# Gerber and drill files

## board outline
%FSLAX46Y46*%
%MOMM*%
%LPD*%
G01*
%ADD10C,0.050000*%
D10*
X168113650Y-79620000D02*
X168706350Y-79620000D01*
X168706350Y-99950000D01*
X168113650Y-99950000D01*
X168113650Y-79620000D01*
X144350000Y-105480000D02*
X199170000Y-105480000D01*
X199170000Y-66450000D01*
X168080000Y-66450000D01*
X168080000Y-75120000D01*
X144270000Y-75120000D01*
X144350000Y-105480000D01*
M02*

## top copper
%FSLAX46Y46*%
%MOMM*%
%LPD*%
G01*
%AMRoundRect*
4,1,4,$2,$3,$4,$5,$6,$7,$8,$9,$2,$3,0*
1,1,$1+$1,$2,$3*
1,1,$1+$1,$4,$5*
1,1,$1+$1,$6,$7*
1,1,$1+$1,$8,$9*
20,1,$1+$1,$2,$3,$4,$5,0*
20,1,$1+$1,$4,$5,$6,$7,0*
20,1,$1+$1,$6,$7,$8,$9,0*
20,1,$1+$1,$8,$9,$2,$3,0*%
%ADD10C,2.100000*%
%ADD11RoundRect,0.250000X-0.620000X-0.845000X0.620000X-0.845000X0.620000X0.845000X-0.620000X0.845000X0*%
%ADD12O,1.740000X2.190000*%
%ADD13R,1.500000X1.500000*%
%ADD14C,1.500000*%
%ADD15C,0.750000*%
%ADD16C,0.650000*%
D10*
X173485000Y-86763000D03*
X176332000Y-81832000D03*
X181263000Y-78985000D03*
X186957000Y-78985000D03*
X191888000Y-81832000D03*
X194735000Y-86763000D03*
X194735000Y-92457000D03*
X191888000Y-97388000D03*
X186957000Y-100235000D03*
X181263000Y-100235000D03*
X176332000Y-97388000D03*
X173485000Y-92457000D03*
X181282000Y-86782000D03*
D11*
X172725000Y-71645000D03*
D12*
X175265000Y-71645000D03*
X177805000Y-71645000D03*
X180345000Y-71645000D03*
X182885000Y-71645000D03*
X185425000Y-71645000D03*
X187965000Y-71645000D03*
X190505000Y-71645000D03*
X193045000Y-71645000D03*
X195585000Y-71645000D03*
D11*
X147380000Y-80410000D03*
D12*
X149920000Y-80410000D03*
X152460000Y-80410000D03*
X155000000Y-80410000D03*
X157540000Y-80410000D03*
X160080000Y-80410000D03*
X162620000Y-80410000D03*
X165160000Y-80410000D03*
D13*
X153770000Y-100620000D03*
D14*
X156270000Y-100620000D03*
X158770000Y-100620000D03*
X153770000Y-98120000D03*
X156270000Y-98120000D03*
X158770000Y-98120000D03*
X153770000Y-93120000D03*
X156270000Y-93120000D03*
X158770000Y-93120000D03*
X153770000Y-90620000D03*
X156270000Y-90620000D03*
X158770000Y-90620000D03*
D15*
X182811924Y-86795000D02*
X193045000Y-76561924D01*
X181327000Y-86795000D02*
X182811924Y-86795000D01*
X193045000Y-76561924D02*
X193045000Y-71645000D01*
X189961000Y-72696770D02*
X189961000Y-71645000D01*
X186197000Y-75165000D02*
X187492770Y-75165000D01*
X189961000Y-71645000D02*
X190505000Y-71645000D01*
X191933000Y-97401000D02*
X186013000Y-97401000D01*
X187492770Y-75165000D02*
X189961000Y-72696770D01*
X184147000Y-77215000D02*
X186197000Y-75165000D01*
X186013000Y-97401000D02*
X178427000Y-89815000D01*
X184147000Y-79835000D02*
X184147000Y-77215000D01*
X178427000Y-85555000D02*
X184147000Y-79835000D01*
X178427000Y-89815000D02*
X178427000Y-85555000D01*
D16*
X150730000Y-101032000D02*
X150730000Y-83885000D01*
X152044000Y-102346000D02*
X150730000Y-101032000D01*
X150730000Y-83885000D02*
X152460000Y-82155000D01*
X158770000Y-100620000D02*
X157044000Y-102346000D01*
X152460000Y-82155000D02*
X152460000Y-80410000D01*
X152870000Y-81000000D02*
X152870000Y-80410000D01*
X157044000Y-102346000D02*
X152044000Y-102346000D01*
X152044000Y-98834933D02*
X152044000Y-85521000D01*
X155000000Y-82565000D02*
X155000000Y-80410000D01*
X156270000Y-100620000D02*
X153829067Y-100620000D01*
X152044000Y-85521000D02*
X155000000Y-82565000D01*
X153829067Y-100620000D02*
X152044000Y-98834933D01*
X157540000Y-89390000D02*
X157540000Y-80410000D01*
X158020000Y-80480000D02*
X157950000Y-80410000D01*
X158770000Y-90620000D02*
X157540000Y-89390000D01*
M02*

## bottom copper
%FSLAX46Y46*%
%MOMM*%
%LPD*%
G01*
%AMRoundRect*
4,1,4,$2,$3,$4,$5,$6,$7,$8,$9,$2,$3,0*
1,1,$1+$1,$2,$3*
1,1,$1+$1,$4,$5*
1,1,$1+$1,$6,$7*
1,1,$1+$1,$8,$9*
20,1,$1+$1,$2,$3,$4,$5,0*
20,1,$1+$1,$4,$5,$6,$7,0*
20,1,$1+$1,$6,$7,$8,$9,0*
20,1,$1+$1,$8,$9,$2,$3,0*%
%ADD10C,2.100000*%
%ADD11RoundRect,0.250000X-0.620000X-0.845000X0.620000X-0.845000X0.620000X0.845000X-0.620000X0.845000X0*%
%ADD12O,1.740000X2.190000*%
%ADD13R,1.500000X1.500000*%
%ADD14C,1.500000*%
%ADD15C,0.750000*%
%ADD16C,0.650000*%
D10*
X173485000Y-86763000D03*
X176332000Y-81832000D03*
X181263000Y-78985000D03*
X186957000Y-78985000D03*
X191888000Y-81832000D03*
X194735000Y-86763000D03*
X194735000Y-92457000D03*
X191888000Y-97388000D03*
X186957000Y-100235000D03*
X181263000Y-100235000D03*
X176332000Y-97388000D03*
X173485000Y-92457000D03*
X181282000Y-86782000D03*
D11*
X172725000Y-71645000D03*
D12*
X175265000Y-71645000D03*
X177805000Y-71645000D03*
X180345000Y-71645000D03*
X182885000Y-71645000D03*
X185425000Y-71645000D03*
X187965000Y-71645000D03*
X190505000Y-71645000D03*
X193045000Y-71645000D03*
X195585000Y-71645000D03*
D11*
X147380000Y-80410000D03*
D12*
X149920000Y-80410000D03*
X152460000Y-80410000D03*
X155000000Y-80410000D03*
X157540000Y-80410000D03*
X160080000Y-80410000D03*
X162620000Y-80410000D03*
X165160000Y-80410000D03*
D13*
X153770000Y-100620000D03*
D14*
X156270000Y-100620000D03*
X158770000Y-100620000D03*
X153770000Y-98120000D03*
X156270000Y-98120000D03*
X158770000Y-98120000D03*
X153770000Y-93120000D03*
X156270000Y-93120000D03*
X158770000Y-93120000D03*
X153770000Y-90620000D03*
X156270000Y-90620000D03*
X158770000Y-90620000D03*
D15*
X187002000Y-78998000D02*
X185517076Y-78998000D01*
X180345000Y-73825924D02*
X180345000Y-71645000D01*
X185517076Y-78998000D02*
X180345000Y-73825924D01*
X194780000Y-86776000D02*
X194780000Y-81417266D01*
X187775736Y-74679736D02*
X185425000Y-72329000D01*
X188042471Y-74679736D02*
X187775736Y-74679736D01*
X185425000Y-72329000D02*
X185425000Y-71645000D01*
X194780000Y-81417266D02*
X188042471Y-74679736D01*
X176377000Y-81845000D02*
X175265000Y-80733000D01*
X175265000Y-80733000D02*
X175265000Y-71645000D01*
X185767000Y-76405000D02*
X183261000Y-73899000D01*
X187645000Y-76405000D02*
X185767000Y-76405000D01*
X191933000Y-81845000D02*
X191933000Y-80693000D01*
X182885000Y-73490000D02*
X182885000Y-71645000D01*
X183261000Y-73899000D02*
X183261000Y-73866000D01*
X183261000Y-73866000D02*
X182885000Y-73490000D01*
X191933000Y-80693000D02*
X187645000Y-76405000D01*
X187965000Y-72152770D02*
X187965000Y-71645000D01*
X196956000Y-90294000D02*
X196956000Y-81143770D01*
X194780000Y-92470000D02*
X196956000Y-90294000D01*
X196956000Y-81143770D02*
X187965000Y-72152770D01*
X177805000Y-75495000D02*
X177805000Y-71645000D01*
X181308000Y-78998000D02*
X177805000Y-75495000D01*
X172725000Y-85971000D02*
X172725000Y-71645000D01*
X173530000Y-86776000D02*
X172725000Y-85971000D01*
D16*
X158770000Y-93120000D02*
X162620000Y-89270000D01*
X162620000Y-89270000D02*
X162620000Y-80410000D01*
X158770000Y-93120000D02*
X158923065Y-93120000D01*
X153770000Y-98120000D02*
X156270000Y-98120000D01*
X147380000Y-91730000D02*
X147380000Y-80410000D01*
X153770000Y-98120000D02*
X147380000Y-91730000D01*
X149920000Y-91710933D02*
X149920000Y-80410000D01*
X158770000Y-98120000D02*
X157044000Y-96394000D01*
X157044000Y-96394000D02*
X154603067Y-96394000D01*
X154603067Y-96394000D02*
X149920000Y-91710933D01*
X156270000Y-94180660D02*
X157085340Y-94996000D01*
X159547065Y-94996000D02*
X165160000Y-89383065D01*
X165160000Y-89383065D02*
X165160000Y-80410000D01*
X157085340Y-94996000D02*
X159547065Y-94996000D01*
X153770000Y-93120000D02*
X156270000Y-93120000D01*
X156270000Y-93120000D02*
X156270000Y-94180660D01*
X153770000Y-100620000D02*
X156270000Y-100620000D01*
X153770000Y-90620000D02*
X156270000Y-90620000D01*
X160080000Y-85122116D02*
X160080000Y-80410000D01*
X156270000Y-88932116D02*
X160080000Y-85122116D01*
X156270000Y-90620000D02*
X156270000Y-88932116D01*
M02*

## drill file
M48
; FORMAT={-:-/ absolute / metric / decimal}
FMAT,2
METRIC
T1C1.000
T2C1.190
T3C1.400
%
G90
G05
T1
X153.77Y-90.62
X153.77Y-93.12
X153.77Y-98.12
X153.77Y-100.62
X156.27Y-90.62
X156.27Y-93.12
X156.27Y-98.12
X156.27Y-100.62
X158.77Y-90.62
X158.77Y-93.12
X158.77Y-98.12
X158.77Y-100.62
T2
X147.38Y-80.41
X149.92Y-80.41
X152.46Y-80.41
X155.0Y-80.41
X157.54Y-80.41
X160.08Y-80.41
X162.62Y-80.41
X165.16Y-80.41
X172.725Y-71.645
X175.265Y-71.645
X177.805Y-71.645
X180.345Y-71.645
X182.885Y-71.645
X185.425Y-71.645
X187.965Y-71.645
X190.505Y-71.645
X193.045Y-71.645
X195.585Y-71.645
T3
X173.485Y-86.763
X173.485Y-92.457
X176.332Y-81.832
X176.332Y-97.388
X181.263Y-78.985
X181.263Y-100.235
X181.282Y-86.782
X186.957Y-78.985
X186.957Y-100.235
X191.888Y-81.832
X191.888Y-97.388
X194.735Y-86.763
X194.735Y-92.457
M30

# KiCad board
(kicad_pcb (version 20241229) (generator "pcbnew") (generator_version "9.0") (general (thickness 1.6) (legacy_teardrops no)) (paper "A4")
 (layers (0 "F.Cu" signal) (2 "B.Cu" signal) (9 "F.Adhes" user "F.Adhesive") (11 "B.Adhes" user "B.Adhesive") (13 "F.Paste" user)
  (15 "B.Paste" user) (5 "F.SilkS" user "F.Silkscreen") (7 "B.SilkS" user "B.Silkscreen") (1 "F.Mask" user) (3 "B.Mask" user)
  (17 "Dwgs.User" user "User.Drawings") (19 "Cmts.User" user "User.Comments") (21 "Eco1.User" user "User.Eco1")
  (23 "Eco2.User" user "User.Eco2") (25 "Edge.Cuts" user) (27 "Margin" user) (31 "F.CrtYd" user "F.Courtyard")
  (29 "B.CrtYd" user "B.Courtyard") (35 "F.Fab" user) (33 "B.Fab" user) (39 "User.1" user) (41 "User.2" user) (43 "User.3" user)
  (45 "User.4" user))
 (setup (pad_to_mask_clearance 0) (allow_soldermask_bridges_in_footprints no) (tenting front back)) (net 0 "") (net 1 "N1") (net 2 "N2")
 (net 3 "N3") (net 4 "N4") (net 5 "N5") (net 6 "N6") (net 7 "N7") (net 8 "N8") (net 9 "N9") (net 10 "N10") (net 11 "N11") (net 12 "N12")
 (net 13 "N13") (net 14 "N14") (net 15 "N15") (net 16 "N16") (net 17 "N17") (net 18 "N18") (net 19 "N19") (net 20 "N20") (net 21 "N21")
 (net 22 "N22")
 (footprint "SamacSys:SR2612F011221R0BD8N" (layer "F.Cu") (at 173.485 86.763)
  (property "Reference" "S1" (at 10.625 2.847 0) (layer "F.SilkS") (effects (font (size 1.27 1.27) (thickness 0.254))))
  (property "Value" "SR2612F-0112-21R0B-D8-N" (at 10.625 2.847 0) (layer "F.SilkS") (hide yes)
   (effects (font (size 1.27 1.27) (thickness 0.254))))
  (pad "1" thru_hole circle (at 0 0) (size 2.1 2.1) (drill 1.4) (layers "*.Cu" "*.Mask") (remove_unused_layers no) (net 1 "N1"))
  (pad "2" thru_hole circle (at 2.847 -4.931) (size 2.1 2.1) (drill 1.4) (layers "*.Cu" "*.Mask") (remove_unused_layers no) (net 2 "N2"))
  (pad "3" thru_hole circle (at 7.778 -7.778) (size 2.1 2.1) (drill 1.4) (layers "*.Cu" "*.Mask") (remove_unused_layers no) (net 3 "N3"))
  (pad "4" thru_hole circle (at 13.472 -7.778) (size 2.1 2.1) (drill 1.4) (layers "*.Cu" "*.Mask") (remove_unused_layers no) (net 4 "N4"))
  (pad "5" thru_hole circle (at 18.403 -4.931) (size 2.1 2.1) (drill 1.4) (layers "*.Cu" "*.Mask") (remove_unused_layers no) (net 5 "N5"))
  (pad "6" thru_hole circle (at 21.25 0) (size 2.1 2.1) (drill 1.4) (layers "*.Cu" "*.Mask") (remove_unused_layers no) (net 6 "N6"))
  (pad "7" thru_hole circle (at 21.25 5.694) (size 2.1 2.1) (drill 1.4) (layers "*.Cu" "*.Mask") (remove_unused_layers no) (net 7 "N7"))
  (pad "8" thru_hole circle (at 18.403 10.625) (size 2.1 2.1) (drill 1.4) (layers "*.Cu" "*.Mask") (remove_unused_layers no) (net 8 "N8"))
  (pad "9" thru_hole circle (at 13.472 13.472) (size 2.1 2.1) (drill 1.4) (layers "*.Cu" "*.Mask") (remove_unused_layers no) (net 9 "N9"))
  (pad "10" thru_hole circle (at 7.778 13.472) (size 2.1 2.1) (drill 1.4) (layers "*.Cu" "*.Mask") (remove_unused_layers no) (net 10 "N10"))
  (pad "11" thru_hole circle (at 2.847 10.625) (size 2.1 2.1) (drill 1.4) (layers "*.Cu" "*.Mask") (remove_unused_layers no) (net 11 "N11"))
  (pad "12" thru_hole circle (at 0 5.694) (size 2.1 2.1) (drill 1.4) (layers "*.Cu" "*.Mask") (remove_unused_layers no) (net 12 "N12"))
  (pad "A1" thru_hole circle (at 7.797 0.019) (size 2.1 2.1) (drill 1.4) (layers "*.Cu" "*.Mask") (remove_unused_layers no) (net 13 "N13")))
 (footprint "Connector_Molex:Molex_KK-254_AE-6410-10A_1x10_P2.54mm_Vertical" (layer "F.Cu") (at 172.725 71.645)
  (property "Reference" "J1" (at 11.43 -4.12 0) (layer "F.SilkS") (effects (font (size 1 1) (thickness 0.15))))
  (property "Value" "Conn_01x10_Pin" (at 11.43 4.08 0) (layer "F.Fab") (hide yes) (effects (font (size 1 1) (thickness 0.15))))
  (pad "1" thru_hole roundrect (at 0 0) (size 1.74 2.19) (drill 1.19) (layers "*.Cu" "*.Mask") (remove_unused_layers no)
   (roundrect_rratio 0.143678) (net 1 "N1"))
  (pad "2" thru_hole oval (at 2.54 0) (size 1.74 2.19) (drill 1.19) (layers "*.Cu" "*.Mask") (remove_unused_layers no) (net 2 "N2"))
  (pad "3" thru_hole oval (at 5.08 0) (size 1.74 2.19) (drill 1.19) (layers "*.Cu" "*.Mask") (remove_unused_layers no) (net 3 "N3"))
  (pad "4" thru_hole oval (at 7.62 0) (size 1.74 2.19) (drill 1.19) (layers "*.Cu" "*.Mask") (remove_unused_layers no) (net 4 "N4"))
  (pad "5" thru_hole oval (at 10.16 0) (size 1.74 2.19) (drill 1.19) (layers "*.Cu" "*.Mask") (remove_unused_layers no) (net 5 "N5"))
  (pad "6" thru_hole oval (at 12.7 0) (size 1.74 2.19) (drill 1.19) (layers "*.Cu" "*.Mask") (remove_unused_layers no) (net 6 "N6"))
  (pad "7" thru_hole oval (at 15.24 0) (size 1.74 2.19) (drill 1.19) (layers "*.Cu" "*.Mask") (remove_unused_layers no) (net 7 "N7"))
  (pad "8" thru_hole oval (at 17.78 0) (size 1.74 2.19) (drill 1.19) (layers "*.Cu" "*.Mask") (remove_unused_layers no) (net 8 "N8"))
  (pad "9" thru_hole oval (at 20.32 0) (size 1.74 2.19) (drill 1.19) (layers "*.Cu" "*.Mask") (remove_unused_layers no) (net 13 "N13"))
  (pad "10" thru_hole oval (at 22.86 0) (size 1.74 2.19) (drill 1.19) (layers "*.Cu" "*.Mask") (remove_unused_layers no) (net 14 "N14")))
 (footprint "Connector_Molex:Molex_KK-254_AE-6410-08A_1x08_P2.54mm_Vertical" (layer "F.Cu") (at 147.38 80.41)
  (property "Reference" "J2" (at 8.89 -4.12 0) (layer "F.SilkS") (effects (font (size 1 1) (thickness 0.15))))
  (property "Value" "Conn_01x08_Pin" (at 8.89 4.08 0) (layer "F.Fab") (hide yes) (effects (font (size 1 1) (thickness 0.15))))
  (pad "1" thru_hole roundrect (at 0 0) (size 1.74 2.19) (drill 1.19) (layers "*.Cu" "*.Mask") (remove_unused_layers no)
   (roundrect_rratio 0.143678) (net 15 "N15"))
  (pad "2" thru_hole oval (at 2.54 0) (size 1.74 2.19) (drill 1.19) (layers "*.Cu" "*.Mask") (remove_unused_layers no) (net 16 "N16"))
  (pad "3" thru_hole oval (at 5.08 0) (size 1.74 2.19) (drill 1.19) (layers "*.Cu" "*.Mask") (remove_unused_layers no) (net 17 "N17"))
  (pad "4" thru_hole oval (at 7.62 0) (size 1.74 2.19) (drill 1.19) (layers "*.Cu" "*.Mask") (remove_unused_layers no) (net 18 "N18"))
  (pad "5" thru_hole oval (at 10.16 0) (size 1.74 2.19) (drill 1.19) (layers "*.Cu" "*.Mask") (remove_unused_layers no) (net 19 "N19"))
  (pad "6" thru_hole oval (at 12.7 0) (size 1.74 2.19) (drill 1.19) (layers "*.Cu" "*.Mask") (remove_unused_layers no) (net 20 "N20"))
  (pad "7" thru_hole oval (at 15.24 0) (size 1.74 2.19) (drill 1.19) (layers "*.Cu" "*.Mask") (remove_unused_layers no) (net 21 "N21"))
  (pad "8" thru_hole oval (at 17.78 0) (size 1.74 2.19) (drill 1.19) (layers "*.Cu" "*.Mask") (remove_unused_layers no) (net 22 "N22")))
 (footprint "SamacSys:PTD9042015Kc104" (layer "F.Cu") (at 153.77 100.62 -90)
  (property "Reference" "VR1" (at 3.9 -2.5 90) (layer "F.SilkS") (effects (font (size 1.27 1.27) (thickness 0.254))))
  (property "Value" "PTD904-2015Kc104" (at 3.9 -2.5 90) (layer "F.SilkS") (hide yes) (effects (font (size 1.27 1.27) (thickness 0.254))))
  (pad "R11" thru_hole rect (at 0 0 270) (size 1.5 1.5) (drill 1) (layers "*.Cu" "*.Mask") (remove_unused_layers no) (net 18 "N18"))
  (pad "R12" thru_hole circle (at 0 -2.5 270) (size 1.5 1.5) (drill 1) (layers "*.Cu" "*.Mask") (remove_unused_layers no) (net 18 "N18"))
  (pad "R13" thru_hole circle (at 0 -5 270) (size 1.5 1.5) (drill 1) (layers "*.Cu" "*.Mask") (remove_unused_layers no) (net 17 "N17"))
  (pad "R21" thru_hole circle (at -2.5 0 270) (size 1.5 1.5) (drill 1) (layers "*.Cu" "*.Mask") (remove_unused_layers no) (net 15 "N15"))
  (pad "R22" thru_hole circle (at -2.5 -2.5 270) (size 1.5 1.5) (drill 1) (layers "*.Cu" "*.Mask") (remove_unused_layers no) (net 15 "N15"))
  (pad "R23" thru_hole circle (at -2.5 -5 270) (size 1.5 1.5) (drill 1) (layers "*.Cu" "*.Mask") (remove_unused_layers no) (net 16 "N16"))
  (pad "R31" thru_hole circle (at -7.5 0 270) (size 1.5 1.5) (drill 1) (layers "*.Cu" "*.Mask") (remove_unused_layers no) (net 22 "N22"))
  (pad "R32" thru_hole circle (at -7.5 -2.5 270) (size 1.5 1.5) (drill 1) (layers "*.Cu" "*.Mask") (remove_unused_layers no) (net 22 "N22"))
  (pad "R33" thru_hole circle (at -7.5 -5 270) (size 1.5 1.5) (drill 1) (layers "*.Cu" "*.Mask") (remove_unused_layers no) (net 21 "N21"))
  (pad "R41" thru_hole circle (at -10 0 270) (size 1.5 1.5) (drill 1) (layers "*.Cu" "*.Mask") (remove_unused_layers no) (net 20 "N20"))
  (pad "R42" thru_hole circle (at -10 -2.5 270) (size 1.5 1.5) (drill 1) (layers "*.Cu" "*.Mask") (remove_unused_layers no) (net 20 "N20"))
  (pad "R43" thru_hole circle (at -10 -5 270) (size 1.5 1.5) (drill 1) (layers "*.Cu" "*.Mask") (remove_unused_layers no) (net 19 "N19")))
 (gr_rect (start 168.11365 79.62) (end 168.70635 99.95) (stroke (width 0.05) (type default)) (fill no) (layer "Edge.Cuts"))
 (gr_poly
  (pts (xy 144.35 105.48) (xy 199.17 105.48) (xy 199.17 66.45) (xy 168.08 66.45) (xy 168.08 75.12) (xy 144.27 75.12))
  (stroke (width 0.05) (type solid)) (fill no) (layer "Edge.Cuts"))
 (segment (start 187.002 78.998) (end 185.517076 78.998) (width 0.75) (layer "B.Cu") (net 4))
 (segment (start 180.345 73.825924) (end 180.345 71.645) (width 0.75) (layer "B.Cu") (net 4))
 (segment (start 185.517076 78.998) (end 180.345 73.825924) (width 0.75) (layer "B.Cu") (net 4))
 (segment (start 194.78 86.776) (end 194.78 81.417266) (width 0.75) (layer "B.Cu") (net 6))
 (segment (start 187.775736 74.679736) (end 185.425 72.329) (width 0.75) (layer "B.Cu") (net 6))
 (segment (start 188.042471 74.679736) (end 187.775736 74.679736) (width 0.75) (layer "B.Cu") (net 6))
 (segment (start 185.425 72.329) (end 185.425 71.645) (width 0.75) (layer "B.Cu") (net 6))
 (segment (start 194.78 81.417266) (end 188.042471 74.679736) (width 0.75) (layer "B.Cu") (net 6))
 (segment (start 182.811924 86.795) (end 193.045 76.561924) (width 0.75) (layer "F.Cu") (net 13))
 (segment (start 181.327 86.795) (end 182.811924 86.795) (width 0.75) (layer "F.Cu") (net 13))
 (segment (start 193.045 76.561924) (end 193.045 71.645) (width 0.75) (layer "F.Cu") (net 13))
 (segment (start 176.377 81.845) (end 175.265 80.733) (width 0.75) (layer "B.Cu") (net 2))
 (segment (start 175.265 80.733) (end 175.265 71.645) (width 0.75) (layer "B.Cu") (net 2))
 (segment (start 185.767 76.405) (end 183.261 73.899) (width 0.75) (layer "B.Cu") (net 5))
 (segment (start 187.645 76.405) (end 185.767 76.405) (width 0.75) (layer "B.Cu") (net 5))
 (segment (start 191.933 81.845) (end 191.933 80.693) (width 0.75) (layer "B.Cu") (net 5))
 (segment (start 182.885 73.49) (end 182.885 71.645) (width 0.75) (layer "B.Cu") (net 5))
 (segment (start 183.261 73.899) (end 183.261 73.866) (width 0.75) (layer "B.Cu") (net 5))
 (segment (start 183.261 73.866) (end 182.885 73.49) (width 0.75) (layer "B.Cu") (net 5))
 (segment (start 191.933 80.693) (end 187.645 76.405) (width 0.75) (layer "B.Cu") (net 5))
 (segment (start 187.965 72.15277) (end 187.965 71.645) (width 0.75) (layer "B.Cu") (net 7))
 (segment (start 196.956 90.294) (end 196.956 81.14377) (width 0.75) (layer "B.Cu") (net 7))
 (segment (start 194.78 92.47) (end 196.956 90.294) (width 0.75) (layer "B.Cu") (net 7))
 (segment (start 196.956 81.14377) (end 187.965 72.15277) (width 0.75) (layer "B.Cu") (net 7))
 (segment (start 177.805 75.495) (end 177.805 71.645) (width 0.75) (layer "B.Cu") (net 3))
 (segment (start 181.308 78.998) (end 177.805 75.495) (width 0.75) (layer "B.Cu") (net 3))
 (segment (start 189.961 72.69677) (end 189.961 71.645) (width 0.75) (layer "F.Cu") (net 8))
 (segment (start 186.197 75.165) (end 187.49277 75.165) (width 0.75) (layer "F.Cu") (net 8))
 (segment (start 189.961 71.645) (end 190.505 71.645) (width 0.75) (layer "F.Cu") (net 8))
 (segment (start 191.933 97.401) (end 186.013 97.401) (width 0.75) (layer "F.Cu") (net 8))
 (segment (start 187.49277 75.165) (end 189.961 72.69677) (width 0.75) (layer "F.Cu") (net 8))
 (segment (start 184.147 77.215) (end 186.197 75.165) (width 0.75) (layer "F.Cu") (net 8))
 (segment (start 186.013 97.401) (end 178.427 89.815) (width 0.75) (layer "F.Cu") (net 8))
 (segment (start 184.147 79.835) (end 184.147 77.215) (width 0.75) (layer "F.Cu") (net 8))
 (segment (start 178.427 85.555) (end 184.147 79.835) (width 0.75) (layer "F.Cu") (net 8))
 (segment (start 178.427 89.815) (end 178.427 85.555) (width 0.75) (layer "F.Cu") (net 8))
 (segment (start 172.725 85.971) (end 172.725 71.645) (width 0.75) (layer "B.Cu") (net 1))
 (segment (start 173.53 86.776) (end 172.725 85.971) (width 0.75) (layer "B.Cu") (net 1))
 (segment (start 158.77 93.12) (end 162.62 89.27) (width 0.65) (layer "B.Cu") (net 21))
 (segment (start 162.62 89.27) (end 162.62 80.41) (width 0.65) (layer "B.Cu") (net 21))
 (segment (start 158.77 93.12) (end 158.923065 93.12) (width 0.65) (layer "B.Cu") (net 21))
 (segment (start 153.77 98.12) (end 156.27 98.12) (width 0.65) (layer "B.Cu") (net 15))
 (segment (start 147.38 91.73) (end 147.38 80.41) (width 0.65) (layer "B.Cu") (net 15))
 (segment (start 153.77 98.12) (end 147.38 91.73) (width 0.65) (layer "B.Cu") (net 15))
 (segment (start 149.92 91.710933) (end 149.92 80.41) (width 0.65) (layer "B.Cu") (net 16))
 (segment (start 158.77 98.12) (end 157.044 96.394) (width 0.65) (layer "B.Cu") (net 16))
 (segment (start 157.044 96.394) (end 154.603067 96.394) (width 0.65) (layer "B.Cu") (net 16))
 (segment (start 154.603067 96.394) (end 149.92 91.710933) (width 0.65) (layer "B.Cu") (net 16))
 (segment (start 156.27 94.18066) (end 157.08534 94.996) (width 0.65) (layer "B.Cu") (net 22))
 (segment (start 159.547065 94.996) (end 165.16 89.383065) (width 0.65) (layer "B.Cu") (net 22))
 (segment (start 165.16 89.383065) (end 165.16 80.41) (width 0.65) (layer "B.Cu") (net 22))
 (segment (start 157.08534 94.996) (end 159.547065 94.996) (width 0.65) (layer "B.Cu") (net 22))
 (segment (start 153.77 93.12) (end 156.27 93.12) (width 0.65) (layer "B.Cu") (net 22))
 (segment (start 156.27 93.12) (end 156.27 94.18066) (width 0.65) (layer "B.Cu") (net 22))
 (segment (start 150.73 101.032) (end 150.73 83.885) (width 0.65) (layer "F.Cu") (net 17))
 (segment (start 152.044 102.346) (end 150.73 101.032) (width 0.65) (layer "F.Cu") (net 17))
 (segment (start 150.73 83.885) (end 152.46 82.155) (width 0.65) (layer "F.Cu") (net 17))
 (segment (start 158.77 100.62) (end 157.044 102.346) (width 0.65) (layer "F.Cu") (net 17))
 (segment (start 152.46 82.155) (end 152.46 80.41) (width 0.65) (layer "F.Cu") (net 17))
 (segment (start 152.87 81) (end 152.87 80.41) (width 0.65) (layer "F.Cu") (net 17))
 (segment (start 157.044 102.346) (end 152.044 102.346) (width 0.65) (layer "F.Cu") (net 17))
 (segment (start 152.044 98.834933) (end 152.044 85.521) (width 0.65) (layer "F.Cu") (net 18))
 (segment (start 155 82.565) (end 155 80.41) (width 0.65) (layer "F.Cu") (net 18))
 (segment (start 156.27 100.62) (end 153.829067 100.62) (width 0.65) (layer "F.Cu") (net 18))
 (segment (start 152.044 85.521) (end 155 82.565) (width 0.65) (layer "F.Cu") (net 18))
 (segment (start 153.829067 100.62) (end 152.044 98.834933) (width 0.65) (layer "F.Cu") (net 18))
 (segment (start 153.77 100.62) (end 156.27 100.62) (width 0.65) (layer "B.Cu") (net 18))
 (segment (start 157.54 89.39) (end 157.54 80.41) (width 0.65) (layer "F.Cu") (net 19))
 (segment (start 158.02 80.48) (end 157.95 80.41) (width 0.65) (layer "F.Cu") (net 19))
 (segment (start 158.77 90.62) (end 157.54 89.39) (width 0.65) (layer "F.Cu") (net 19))
 (segment (start 153.77 90.62) (end 156.27 90.62) (width 0.65) (layer "B.Cu") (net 20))
 (segment (start 160.08 85.122116) (end 160.08 80.41) (width 0.65) (layer "B.Cu") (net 20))
 (segment (start 156.27 88.932116) (end 160.08 85.122116) (width 0.65) (layer "B.Cu") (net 20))
 (segment (start 156.27 90.62) (end 156.27 88.932116) (width 0.65) (layer "B.Cu") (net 20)))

